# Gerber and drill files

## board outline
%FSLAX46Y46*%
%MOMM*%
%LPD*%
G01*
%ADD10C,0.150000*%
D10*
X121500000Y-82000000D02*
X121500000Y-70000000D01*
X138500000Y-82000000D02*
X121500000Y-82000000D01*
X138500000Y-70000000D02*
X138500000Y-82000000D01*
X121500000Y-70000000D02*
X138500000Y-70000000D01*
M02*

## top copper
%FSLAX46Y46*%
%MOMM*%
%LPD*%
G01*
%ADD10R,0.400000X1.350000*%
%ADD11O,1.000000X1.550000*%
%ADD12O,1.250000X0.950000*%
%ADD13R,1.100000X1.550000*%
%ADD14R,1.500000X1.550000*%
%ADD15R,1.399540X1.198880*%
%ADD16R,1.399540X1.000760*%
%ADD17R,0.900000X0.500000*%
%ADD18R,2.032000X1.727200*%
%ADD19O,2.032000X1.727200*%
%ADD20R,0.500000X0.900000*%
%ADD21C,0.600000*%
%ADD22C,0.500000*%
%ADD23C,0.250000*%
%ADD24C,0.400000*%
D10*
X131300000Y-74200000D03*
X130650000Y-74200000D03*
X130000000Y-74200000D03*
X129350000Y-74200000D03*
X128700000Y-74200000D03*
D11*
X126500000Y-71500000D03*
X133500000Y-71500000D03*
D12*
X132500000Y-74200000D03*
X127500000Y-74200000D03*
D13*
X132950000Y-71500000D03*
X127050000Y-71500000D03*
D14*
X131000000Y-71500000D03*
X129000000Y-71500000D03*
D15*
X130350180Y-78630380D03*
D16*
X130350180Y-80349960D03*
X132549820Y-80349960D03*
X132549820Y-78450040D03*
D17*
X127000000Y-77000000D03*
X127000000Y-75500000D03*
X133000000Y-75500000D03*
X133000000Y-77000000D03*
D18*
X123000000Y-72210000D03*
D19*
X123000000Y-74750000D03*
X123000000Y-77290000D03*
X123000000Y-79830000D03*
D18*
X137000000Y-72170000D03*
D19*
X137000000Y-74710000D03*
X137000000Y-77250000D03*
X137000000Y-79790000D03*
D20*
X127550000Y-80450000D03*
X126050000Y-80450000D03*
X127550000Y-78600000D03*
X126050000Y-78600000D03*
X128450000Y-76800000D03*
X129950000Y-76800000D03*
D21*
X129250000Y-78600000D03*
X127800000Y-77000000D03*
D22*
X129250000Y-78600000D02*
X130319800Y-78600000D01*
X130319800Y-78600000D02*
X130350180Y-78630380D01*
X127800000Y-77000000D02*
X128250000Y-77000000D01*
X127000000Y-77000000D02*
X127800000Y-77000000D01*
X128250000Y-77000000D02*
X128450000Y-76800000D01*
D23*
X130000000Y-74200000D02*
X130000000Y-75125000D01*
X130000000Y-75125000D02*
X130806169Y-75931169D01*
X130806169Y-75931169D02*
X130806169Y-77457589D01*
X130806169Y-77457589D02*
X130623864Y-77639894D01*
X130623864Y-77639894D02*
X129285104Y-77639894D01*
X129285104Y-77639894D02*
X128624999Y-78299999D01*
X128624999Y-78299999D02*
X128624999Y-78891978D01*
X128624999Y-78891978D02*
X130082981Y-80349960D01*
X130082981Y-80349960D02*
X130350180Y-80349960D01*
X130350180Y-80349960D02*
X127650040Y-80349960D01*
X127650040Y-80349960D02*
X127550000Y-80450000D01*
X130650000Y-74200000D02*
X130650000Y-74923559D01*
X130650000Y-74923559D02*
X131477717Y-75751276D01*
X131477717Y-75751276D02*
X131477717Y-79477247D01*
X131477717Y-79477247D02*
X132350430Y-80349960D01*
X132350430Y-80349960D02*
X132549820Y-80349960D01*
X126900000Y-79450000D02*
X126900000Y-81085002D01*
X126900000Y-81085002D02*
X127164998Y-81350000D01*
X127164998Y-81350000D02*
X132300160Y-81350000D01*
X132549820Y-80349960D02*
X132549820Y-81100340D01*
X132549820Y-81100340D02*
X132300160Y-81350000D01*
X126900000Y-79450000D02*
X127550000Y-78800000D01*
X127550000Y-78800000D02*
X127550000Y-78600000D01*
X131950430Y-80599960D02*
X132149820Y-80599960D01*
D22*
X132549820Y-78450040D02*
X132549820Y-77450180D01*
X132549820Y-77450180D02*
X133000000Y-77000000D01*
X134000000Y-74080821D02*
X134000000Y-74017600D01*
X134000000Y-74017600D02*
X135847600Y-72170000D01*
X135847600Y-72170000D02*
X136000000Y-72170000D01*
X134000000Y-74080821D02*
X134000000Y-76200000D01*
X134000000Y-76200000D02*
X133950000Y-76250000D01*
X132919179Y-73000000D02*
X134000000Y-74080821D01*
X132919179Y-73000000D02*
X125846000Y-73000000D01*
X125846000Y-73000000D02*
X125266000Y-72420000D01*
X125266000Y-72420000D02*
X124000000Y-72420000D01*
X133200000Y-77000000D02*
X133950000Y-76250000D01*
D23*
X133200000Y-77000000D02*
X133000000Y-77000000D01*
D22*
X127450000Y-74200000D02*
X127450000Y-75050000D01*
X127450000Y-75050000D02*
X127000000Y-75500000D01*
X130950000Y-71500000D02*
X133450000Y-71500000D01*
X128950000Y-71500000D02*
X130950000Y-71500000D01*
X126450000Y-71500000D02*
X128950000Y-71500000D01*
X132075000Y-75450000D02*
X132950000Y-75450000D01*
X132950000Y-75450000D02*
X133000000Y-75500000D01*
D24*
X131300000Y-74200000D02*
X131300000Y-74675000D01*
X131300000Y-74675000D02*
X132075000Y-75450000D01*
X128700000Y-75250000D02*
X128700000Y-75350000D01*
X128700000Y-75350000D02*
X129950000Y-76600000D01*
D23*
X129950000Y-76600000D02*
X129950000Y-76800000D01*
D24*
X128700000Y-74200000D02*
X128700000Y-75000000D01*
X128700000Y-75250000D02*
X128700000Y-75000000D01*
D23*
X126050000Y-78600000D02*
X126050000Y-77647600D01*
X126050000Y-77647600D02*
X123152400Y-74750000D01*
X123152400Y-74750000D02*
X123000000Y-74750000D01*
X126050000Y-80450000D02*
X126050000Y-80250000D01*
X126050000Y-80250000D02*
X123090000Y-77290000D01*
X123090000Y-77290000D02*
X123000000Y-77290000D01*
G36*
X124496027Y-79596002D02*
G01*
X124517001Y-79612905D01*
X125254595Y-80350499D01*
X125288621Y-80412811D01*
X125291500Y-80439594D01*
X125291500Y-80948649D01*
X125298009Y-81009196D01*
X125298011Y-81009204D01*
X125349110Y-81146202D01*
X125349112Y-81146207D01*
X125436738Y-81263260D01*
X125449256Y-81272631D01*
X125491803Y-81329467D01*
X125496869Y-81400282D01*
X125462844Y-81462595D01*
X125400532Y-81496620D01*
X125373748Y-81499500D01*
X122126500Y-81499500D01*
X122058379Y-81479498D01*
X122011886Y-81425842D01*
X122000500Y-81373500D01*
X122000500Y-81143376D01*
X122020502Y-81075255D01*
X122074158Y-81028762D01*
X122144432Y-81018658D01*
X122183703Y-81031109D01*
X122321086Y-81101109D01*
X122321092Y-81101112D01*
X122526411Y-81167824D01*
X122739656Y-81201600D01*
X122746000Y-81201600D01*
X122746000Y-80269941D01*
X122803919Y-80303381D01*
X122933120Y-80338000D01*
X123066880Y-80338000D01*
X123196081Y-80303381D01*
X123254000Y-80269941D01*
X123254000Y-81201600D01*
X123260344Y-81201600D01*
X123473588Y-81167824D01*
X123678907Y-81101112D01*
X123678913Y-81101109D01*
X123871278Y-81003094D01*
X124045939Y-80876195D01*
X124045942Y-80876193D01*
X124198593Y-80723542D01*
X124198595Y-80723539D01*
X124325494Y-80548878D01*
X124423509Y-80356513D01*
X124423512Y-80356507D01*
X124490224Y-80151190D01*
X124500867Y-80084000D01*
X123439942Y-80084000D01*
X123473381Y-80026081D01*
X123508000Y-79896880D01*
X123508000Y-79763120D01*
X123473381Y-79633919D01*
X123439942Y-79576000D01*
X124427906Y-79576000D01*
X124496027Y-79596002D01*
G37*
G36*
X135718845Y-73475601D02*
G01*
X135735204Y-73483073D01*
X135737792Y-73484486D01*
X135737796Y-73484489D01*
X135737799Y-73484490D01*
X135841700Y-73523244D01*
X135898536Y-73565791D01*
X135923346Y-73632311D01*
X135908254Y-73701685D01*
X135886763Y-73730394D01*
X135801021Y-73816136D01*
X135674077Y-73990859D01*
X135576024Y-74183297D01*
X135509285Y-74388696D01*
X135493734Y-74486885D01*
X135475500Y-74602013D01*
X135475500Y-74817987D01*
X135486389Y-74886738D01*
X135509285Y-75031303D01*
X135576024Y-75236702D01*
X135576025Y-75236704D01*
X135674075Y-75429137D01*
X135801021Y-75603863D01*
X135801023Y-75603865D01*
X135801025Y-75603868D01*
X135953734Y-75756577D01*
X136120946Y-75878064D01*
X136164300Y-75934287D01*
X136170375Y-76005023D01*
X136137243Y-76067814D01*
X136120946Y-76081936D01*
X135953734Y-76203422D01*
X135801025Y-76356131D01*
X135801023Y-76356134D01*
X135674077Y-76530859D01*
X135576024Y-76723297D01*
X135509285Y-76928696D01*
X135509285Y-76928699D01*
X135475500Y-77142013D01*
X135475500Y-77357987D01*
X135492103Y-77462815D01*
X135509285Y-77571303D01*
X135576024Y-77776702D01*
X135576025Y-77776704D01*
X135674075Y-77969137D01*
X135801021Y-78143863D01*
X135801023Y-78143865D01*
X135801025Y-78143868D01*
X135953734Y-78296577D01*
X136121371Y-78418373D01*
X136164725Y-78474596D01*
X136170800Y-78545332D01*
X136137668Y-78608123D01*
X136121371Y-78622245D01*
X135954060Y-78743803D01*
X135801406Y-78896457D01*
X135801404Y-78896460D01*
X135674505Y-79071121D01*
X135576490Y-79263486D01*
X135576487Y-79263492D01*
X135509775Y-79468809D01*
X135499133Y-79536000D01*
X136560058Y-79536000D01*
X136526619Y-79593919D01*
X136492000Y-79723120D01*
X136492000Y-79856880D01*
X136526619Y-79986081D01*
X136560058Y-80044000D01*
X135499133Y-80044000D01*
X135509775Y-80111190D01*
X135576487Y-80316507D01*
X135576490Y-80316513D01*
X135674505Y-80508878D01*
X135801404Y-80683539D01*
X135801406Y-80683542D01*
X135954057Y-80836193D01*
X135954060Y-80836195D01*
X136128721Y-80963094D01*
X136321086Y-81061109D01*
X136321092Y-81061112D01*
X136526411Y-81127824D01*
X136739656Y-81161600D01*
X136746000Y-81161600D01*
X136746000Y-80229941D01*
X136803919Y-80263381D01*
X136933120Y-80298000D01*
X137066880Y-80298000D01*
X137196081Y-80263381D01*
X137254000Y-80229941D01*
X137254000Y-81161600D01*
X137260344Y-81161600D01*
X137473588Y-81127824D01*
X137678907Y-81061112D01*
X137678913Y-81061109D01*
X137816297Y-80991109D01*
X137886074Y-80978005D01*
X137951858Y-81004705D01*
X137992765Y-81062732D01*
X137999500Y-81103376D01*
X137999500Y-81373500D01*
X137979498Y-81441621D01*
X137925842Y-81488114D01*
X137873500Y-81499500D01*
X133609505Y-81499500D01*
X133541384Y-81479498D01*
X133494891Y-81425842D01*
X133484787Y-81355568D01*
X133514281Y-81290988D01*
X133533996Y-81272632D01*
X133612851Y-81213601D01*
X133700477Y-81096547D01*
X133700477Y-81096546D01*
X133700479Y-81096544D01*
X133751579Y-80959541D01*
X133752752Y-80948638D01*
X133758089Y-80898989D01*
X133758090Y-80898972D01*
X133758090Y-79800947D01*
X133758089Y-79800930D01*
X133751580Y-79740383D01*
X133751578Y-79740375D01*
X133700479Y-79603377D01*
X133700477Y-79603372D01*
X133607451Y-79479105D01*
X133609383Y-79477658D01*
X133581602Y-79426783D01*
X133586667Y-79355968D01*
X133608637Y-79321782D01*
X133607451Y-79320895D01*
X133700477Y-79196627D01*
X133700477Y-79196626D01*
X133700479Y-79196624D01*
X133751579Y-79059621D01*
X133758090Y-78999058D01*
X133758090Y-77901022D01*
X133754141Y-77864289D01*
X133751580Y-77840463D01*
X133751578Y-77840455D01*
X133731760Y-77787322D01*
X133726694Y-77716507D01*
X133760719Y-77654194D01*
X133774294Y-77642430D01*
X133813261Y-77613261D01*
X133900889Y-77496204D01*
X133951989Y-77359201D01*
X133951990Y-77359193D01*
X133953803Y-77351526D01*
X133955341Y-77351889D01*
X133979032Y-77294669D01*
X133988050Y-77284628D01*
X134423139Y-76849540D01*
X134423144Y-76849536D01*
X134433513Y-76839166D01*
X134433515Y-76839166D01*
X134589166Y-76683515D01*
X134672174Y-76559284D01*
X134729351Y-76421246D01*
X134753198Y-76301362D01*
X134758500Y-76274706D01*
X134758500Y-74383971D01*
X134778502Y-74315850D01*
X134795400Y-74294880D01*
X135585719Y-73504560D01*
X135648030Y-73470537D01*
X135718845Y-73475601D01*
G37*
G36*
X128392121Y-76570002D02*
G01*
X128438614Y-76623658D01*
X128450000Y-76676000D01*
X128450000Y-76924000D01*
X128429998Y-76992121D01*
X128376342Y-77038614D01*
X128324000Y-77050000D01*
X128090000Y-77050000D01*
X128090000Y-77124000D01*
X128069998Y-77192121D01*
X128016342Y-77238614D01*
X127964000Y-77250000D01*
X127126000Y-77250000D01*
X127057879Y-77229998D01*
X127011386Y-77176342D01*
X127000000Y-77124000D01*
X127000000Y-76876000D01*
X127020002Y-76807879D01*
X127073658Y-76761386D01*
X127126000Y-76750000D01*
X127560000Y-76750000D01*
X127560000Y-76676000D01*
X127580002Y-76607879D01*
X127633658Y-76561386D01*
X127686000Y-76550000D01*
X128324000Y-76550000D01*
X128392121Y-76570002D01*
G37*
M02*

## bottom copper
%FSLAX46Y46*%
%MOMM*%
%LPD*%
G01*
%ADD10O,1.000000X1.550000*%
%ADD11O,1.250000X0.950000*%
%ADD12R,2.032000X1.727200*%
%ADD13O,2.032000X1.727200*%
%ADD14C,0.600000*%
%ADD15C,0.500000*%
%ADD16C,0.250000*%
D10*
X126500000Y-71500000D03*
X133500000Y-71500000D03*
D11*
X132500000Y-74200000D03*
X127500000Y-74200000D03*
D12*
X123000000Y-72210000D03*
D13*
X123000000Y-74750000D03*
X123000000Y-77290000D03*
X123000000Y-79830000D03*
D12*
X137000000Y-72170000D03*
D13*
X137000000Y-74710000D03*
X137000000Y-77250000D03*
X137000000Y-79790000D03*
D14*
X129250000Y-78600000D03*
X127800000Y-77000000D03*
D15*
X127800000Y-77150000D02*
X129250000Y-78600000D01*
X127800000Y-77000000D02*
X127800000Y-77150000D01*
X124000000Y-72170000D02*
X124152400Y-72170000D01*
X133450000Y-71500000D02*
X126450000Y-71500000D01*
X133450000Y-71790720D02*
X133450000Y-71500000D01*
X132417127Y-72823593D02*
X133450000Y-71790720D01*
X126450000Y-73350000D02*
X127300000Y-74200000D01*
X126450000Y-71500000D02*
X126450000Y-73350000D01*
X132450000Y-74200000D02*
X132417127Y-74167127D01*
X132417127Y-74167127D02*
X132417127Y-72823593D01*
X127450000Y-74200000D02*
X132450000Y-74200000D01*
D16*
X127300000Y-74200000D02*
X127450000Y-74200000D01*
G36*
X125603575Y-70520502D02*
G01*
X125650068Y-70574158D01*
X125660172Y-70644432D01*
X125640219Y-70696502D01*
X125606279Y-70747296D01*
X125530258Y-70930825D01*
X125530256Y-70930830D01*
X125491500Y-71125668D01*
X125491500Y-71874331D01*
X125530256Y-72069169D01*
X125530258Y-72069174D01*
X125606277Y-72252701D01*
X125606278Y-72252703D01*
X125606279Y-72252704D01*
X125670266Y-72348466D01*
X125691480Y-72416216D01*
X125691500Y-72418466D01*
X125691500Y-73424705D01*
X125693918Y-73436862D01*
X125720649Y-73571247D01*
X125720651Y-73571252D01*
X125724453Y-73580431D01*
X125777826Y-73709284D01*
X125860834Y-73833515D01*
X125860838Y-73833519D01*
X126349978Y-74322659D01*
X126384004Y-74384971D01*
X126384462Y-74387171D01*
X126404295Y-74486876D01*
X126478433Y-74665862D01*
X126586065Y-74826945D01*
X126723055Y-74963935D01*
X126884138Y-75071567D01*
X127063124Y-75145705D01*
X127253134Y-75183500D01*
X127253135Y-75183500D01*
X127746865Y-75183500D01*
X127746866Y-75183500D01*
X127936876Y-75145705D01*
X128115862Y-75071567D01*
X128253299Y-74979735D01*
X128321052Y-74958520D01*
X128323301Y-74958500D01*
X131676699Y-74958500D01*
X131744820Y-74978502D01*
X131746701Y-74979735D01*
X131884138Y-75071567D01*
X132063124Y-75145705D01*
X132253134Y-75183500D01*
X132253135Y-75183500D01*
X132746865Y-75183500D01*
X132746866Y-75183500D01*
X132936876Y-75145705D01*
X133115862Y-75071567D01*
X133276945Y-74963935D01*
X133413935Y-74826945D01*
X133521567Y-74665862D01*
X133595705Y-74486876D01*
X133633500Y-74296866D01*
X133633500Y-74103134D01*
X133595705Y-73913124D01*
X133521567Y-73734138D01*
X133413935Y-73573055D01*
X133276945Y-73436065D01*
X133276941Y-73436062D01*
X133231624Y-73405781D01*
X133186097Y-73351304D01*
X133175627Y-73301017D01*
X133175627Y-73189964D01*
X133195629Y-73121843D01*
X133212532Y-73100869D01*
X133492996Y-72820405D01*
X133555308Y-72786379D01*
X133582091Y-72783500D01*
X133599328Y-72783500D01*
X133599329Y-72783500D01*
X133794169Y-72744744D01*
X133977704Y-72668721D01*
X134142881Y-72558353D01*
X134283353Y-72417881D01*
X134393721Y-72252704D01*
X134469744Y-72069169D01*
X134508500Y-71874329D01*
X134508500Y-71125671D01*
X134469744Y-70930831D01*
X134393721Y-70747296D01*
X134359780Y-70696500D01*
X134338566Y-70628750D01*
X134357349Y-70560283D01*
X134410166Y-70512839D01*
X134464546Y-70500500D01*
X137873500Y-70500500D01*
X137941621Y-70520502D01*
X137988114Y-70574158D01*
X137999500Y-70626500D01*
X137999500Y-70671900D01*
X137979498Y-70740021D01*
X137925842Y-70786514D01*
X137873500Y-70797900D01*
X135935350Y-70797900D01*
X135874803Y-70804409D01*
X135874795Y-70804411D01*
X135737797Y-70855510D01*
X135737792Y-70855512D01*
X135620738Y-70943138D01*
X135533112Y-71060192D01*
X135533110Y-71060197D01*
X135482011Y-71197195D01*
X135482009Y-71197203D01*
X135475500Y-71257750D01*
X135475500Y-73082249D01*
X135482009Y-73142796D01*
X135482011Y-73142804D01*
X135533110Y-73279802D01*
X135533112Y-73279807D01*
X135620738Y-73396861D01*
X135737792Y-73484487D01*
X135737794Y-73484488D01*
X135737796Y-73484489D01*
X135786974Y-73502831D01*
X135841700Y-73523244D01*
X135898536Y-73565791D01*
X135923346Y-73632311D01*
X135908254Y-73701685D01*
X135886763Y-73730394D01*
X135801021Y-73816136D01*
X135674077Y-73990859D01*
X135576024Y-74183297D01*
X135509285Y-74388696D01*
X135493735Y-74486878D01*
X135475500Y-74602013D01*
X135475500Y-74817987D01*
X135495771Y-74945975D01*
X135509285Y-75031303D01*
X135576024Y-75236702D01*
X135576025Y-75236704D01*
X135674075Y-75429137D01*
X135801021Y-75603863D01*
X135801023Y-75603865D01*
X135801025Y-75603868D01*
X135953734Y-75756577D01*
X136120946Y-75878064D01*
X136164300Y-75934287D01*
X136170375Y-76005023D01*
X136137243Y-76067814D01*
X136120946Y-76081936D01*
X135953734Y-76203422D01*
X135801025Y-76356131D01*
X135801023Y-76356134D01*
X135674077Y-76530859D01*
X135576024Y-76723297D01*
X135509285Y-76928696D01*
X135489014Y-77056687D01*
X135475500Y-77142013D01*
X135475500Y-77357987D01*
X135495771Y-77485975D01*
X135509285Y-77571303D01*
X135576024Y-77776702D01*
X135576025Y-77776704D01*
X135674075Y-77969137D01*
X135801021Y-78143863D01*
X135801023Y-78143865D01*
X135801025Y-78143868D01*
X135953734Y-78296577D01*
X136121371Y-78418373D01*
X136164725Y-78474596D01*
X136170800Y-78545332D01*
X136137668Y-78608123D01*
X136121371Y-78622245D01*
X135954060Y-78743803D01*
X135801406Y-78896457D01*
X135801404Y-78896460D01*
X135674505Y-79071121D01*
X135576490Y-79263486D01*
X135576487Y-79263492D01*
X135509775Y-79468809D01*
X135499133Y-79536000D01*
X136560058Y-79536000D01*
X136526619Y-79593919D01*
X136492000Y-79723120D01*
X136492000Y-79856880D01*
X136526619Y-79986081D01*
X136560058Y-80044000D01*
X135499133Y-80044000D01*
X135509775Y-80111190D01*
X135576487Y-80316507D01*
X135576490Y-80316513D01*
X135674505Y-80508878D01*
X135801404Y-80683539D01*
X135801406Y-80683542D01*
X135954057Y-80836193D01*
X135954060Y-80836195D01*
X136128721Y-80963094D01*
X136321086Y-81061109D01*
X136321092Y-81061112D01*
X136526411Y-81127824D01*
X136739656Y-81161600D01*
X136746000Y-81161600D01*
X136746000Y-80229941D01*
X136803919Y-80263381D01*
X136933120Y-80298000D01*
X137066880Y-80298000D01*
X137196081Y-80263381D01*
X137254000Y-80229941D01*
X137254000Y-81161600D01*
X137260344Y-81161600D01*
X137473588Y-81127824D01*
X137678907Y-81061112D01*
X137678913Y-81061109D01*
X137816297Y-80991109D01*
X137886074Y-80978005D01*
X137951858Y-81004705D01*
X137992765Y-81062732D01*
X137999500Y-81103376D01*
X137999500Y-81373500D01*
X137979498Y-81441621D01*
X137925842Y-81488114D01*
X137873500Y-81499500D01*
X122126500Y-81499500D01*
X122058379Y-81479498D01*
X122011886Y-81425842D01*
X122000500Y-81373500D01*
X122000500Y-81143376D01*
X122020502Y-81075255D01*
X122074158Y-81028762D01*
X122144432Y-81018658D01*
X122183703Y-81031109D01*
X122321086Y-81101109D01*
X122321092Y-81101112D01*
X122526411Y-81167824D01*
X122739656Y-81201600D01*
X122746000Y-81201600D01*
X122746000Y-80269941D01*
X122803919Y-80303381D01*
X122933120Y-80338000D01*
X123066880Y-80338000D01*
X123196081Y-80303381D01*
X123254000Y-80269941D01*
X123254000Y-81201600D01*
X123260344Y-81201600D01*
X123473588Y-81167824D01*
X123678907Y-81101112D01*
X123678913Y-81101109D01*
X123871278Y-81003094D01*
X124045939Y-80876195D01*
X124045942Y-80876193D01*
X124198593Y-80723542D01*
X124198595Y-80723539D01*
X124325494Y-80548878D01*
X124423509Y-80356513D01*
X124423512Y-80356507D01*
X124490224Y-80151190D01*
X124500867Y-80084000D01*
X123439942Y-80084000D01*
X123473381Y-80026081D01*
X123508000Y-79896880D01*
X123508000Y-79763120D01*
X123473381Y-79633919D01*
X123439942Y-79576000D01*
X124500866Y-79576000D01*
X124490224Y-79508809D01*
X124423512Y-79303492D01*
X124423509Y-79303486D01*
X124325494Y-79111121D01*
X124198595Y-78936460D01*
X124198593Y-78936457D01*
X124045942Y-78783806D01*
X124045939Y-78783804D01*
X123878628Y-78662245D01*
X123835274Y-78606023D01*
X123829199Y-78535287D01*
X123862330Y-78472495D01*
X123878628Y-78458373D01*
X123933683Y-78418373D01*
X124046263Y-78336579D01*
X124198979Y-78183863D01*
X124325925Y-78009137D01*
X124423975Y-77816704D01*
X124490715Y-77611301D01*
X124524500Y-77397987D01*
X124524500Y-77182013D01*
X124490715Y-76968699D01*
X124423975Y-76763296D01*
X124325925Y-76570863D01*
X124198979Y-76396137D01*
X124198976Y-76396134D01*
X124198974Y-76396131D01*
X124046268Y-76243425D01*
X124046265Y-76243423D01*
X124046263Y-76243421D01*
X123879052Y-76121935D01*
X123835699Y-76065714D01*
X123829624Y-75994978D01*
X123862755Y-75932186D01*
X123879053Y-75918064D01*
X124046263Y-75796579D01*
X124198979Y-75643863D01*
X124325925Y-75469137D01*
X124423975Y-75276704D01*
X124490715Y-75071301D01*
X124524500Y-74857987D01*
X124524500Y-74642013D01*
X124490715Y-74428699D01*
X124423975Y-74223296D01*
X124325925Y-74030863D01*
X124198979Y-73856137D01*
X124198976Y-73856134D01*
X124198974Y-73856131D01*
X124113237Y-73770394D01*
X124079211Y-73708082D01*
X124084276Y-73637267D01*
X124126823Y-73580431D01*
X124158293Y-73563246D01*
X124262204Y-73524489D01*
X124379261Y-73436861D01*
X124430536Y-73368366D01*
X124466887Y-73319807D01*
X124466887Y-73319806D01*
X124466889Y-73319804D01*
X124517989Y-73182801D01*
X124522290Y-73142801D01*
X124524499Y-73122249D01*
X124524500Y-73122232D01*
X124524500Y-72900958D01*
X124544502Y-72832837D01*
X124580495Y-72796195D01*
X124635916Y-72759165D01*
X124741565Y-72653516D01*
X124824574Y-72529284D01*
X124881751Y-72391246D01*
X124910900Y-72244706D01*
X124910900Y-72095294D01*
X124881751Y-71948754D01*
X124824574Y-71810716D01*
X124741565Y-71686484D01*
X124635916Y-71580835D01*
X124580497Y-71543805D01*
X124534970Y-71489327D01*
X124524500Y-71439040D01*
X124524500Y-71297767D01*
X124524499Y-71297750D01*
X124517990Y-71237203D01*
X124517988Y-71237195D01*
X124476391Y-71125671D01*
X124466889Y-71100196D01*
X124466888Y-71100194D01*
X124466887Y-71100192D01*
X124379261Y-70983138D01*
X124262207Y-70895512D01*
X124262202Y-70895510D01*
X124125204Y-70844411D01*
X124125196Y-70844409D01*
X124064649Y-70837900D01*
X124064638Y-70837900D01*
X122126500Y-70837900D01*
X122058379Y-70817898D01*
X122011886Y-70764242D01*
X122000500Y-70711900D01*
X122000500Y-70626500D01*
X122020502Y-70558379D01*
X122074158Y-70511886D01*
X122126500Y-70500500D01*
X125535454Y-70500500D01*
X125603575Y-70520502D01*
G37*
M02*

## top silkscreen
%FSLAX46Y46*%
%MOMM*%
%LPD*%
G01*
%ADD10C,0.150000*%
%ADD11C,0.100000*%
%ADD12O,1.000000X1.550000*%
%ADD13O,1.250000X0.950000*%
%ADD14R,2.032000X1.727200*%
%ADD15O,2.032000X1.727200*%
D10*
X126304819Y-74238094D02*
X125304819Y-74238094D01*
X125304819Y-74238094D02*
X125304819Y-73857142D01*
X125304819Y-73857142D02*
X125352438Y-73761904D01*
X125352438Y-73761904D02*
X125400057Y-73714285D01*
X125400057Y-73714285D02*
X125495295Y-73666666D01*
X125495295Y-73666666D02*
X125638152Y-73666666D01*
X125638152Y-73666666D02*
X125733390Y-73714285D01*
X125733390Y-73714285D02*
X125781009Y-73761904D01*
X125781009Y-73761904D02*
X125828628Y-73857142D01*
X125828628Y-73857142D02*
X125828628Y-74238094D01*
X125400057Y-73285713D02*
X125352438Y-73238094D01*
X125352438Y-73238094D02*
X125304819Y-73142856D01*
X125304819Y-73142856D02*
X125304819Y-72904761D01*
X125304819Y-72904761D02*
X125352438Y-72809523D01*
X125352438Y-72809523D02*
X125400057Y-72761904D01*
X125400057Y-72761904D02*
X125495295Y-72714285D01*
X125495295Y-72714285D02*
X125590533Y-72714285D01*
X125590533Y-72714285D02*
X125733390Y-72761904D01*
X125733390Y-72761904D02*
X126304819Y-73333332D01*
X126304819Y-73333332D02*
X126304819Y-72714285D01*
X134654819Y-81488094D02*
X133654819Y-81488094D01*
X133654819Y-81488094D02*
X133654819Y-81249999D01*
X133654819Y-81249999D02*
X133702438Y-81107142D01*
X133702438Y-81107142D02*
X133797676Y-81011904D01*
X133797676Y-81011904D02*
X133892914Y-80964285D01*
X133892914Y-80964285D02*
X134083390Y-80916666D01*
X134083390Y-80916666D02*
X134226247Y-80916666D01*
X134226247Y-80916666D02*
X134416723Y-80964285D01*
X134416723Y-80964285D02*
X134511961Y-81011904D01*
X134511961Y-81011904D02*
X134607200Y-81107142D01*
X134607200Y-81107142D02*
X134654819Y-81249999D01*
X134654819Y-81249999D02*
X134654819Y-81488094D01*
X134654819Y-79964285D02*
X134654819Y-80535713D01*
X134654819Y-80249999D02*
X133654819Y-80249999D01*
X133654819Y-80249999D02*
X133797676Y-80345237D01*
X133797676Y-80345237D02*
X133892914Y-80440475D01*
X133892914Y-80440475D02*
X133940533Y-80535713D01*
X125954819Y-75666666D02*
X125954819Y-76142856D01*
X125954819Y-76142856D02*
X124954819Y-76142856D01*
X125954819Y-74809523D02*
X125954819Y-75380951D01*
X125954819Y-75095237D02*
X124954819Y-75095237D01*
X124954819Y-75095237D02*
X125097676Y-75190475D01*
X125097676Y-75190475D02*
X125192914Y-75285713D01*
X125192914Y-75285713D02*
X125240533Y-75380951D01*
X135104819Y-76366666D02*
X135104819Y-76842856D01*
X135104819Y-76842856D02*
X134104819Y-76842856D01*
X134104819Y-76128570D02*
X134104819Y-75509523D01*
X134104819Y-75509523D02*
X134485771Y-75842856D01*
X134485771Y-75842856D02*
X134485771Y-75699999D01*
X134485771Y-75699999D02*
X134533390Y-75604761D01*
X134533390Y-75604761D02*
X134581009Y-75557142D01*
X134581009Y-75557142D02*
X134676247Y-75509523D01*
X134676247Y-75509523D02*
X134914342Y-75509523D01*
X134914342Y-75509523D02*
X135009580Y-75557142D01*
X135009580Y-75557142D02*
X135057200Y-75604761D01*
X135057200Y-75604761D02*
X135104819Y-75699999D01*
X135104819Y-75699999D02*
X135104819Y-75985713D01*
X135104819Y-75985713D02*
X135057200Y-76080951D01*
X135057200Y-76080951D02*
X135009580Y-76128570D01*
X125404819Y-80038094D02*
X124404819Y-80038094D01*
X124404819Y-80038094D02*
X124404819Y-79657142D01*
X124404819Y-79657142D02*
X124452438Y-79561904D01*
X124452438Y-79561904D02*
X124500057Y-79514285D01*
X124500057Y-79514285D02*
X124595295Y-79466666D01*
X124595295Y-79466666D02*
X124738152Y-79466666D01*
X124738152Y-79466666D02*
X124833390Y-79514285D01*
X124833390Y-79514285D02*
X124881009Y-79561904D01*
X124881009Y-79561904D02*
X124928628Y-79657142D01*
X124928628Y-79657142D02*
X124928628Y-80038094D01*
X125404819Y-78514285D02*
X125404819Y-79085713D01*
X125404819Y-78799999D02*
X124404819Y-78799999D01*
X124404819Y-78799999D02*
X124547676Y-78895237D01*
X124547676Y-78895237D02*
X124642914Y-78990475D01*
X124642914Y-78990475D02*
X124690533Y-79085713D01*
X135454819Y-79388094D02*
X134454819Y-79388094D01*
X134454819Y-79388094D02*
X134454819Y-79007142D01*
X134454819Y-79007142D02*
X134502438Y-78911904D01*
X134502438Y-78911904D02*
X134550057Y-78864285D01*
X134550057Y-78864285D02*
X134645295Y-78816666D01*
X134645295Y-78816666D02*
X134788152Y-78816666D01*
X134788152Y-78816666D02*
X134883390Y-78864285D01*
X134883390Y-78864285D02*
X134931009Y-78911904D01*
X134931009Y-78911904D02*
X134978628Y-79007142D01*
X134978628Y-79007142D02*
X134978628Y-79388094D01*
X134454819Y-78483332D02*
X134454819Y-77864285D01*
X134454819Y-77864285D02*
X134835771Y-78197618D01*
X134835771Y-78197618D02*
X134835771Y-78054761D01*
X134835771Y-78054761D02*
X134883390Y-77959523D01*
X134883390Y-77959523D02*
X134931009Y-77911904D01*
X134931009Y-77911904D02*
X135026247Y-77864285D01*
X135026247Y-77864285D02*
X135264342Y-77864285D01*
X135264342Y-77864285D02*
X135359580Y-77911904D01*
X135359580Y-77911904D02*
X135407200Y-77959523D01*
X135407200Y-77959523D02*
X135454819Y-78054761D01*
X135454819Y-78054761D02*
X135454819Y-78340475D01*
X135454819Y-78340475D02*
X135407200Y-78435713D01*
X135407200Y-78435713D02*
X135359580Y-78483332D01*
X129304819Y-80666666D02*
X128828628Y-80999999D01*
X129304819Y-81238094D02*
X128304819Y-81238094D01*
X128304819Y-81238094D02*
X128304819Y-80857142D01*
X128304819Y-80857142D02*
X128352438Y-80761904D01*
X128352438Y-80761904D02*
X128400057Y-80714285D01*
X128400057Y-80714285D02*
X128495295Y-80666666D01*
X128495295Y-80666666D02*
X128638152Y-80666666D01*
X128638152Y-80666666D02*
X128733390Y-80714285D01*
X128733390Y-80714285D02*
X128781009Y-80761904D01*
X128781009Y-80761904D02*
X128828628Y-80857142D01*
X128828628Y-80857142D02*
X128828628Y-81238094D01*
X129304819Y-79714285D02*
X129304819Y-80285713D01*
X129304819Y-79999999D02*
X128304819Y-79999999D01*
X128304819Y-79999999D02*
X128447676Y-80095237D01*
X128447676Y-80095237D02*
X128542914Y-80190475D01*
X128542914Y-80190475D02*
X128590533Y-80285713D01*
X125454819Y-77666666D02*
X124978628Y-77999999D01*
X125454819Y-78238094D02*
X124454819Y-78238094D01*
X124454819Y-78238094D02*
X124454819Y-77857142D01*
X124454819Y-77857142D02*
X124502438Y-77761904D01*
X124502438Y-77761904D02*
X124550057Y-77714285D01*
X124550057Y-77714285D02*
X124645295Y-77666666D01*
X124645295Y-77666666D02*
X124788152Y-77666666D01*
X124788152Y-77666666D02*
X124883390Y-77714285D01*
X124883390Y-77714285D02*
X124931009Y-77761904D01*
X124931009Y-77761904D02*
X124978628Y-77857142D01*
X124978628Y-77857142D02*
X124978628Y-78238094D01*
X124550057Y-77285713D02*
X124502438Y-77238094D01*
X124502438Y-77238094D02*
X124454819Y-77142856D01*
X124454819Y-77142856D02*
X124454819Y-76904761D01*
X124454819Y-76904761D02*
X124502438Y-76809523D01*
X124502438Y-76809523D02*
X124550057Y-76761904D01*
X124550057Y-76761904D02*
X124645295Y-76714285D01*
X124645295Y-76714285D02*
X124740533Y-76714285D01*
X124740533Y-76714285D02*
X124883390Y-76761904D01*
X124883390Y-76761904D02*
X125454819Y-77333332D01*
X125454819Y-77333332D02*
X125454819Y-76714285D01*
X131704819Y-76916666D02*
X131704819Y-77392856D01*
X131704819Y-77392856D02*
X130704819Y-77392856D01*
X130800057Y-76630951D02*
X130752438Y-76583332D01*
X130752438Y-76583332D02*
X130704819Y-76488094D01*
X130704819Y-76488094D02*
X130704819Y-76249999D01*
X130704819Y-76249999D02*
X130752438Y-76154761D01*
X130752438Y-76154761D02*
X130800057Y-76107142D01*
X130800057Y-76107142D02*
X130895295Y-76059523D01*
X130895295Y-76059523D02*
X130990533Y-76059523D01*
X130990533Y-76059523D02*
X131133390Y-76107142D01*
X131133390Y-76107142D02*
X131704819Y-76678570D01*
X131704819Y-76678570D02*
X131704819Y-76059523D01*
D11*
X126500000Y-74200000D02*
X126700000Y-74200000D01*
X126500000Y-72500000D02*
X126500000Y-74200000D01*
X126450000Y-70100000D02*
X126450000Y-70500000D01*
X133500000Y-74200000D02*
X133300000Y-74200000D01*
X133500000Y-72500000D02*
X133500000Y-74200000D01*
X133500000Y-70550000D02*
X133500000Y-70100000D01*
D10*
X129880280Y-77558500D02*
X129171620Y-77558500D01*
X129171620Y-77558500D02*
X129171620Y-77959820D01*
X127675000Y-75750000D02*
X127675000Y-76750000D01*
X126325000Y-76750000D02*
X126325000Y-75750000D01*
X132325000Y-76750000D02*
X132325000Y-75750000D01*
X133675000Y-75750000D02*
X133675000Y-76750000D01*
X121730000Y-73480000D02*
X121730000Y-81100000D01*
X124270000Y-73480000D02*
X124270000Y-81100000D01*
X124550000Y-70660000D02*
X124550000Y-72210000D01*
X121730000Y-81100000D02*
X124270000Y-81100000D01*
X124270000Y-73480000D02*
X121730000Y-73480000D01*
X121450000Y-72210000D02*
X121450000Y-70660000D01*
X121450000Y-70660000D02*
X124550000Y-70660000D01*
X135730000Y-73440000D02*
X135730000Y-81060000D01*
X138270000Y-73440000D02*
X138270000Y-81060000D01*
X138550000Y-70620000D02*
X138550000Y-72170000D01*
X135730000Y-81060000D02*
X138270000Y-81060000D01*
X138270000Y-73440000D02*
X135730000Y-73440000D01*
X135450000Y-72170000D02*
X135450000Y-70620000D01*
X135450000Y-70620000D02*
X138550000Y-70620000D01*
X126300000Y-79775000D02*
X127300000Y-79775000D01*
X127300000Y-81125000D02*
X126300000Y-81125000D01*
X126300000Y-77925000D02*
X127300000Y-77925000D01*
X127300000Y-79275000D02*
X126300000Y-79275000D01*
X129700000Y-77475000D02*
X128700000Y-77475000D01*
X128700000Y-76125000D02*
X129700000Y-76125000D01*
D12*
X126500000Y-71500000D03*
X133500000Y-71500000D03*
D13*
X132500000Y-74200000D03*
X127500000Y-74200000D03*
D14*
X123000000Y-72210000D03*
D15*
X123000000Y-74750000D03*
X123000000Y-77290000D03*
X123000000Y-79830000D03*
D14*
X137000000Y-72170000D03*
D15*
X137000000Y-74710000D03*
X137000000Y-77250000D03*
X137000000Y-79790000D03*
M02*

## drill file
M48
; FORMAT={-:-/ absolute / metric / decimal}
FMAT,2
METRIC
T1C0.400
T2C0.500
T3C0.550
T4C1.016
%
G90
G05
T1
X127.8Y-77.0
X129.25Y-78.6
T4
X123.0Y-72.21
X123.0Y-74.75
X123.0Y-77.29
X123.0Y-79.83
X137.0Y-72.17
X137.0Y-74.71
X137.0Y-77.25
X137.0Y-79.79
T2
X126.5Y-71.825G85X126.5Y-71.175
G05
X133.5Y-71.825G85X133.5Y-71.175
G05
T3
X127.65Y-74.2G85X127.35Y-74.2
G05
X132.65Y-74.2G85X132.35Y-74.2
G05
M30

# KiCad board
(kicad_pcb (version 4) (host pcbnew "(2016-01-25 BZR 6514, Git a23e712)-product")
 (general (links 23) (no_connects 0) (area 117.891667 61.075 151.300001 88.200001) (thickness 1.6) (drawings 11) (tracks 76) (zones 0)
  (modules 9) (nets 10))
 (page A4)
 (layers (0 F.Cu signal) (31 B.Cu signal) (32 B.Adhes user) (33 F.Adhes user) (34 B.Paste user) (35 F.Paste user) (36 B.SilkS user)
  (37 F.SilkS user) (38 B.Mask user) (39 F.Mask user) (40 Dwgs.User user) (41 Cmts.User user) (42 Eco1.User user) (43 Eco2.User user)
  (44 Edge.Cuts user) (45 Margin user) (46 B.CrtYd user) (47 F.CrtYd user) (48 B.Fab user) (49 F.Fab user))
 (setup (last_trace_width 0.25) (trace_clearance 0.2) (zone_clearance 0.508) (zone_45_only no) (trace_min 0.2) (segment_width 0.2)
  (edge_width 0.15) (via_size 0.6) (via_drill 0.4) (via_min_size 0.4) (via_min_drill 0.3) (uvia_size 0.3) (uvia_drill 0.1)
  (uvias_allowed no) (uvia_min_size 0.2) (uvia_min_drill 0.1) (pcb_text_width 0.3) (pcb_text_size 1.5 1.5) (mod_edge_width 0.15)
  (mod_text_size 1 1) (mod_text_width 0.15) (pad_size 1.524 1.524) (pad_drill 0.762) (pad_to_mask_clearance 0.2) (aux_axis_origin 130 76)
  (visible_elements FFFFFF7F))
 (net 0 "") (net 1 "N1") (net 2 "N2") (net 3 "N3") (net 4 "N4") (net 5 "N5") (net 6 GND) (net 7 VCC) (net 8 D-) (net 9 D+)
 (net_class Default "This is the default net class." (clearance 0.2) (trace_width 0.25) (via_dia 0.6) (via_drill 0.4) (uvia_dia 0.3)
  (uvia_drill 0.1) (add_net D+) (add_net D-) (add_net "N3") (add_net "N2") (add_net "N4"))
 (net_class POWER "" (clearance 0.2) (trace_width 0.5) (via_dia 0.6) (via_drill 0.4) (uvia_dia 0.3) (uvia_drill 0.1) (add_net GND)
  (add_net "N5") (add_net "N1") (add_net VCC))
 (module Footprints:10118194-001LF (layer F.Cu) (at 130 71.5 180)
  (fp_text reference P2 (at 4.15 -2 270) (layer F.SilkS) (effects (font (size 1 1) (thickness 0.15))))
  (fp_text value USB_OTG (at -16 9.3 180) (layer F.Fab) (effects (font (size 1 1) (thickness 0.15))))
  (fp_line (start 3.5 -2.7) (end 3.3 -2.7) (layer F.SilkS) (width 0.1))
  (fp_line (start 3.5 -1) (end 3.5 -2.7) (layer F.SilkS) (width 0.1))
  (fp_line (start 3.55 1.4) (end 3.55 1) (layer F.SilkS) (width 0.1))
  (fp_line (start -3.5 -2.7) (end -3.3 -2.7) (layer F.SilkS) (width 0.1))
  (fp_line (start -3.5 -1) (end -3.5 -2.7) (layer F.SilkS) (width 0.1))
  (fp_line (start -3.5 0.95) (end -3.5 1.4) (layer F.SilkS) (width 0.1))
  (pad 1 smd rect (at -1.3 -2.7 180) (size 0.4 1.35) (layers F.Cu F.Paste F.Mask) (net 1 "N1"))
  (pad 2 smd rect (at -0.65 -2.7 180) (size 0.4 1.35) (layers F.Cu F.Paste F.Mask) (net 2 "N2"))
  (pad 3 smd rect (at 0 -2.7 180) (size 0.4 1.35) (layers F.Cu F.Paste F.Mask) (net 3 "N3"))
  (pad 4 smd rect (at 0.65 -2.7 180) (size 0.4 1.35) (layers F.Cu F.Paste F.Mask))
  (pad 5 smd rect (at 1.3 -2.7 180) (size 0.4 1.35) (layers F.Cu F.Paste F.Mask) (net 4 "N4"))
  (pad 6 thru_hole oval (at 3.5 0 180) (size 1 1.55) (drill oval 0.5 1.15) (layers *.Cu *.Mask F.SilkS) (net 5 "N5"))
  (pad 6 thru_hole oval (at -3.5 0 180) (size 1 1.55) (drill oval 0.5 1.15) (layers *.Cu *.Mask F.SilkS) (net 5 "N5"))
  (pad 6 thru_hole oval (at -2.5 -2.7 180) (size 1.25 0.95) (drill oval 0.85 0.55) (layers *.Cu *.Mask F.SilkS) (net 5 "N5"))
  (pad 6 thru_hole oval (at 2.5 -2.7 180) (size 1.25 0.95) (drill oval 0.85 0.55) (layers *.Cu *.Mask F.SilkS) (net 5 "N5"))
  (pad 6 smd rect (at -2.95 0 270) (size 1.55 1.1) (layers F.Cu F.Paste F.Mask) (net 5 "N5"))
  (pad 6 smd rect (at 2.95 0 270) (size 1.55 1.1) (layers F.Cu F.Paste F.Mask) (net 5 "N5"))
  (pad 6 smd rect (at -1 0 270) (size 1.55 1.5) (layers F.Cu F.Paste F.Mask) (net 5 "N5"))
  (pad 6 smd rect (at 1 0 270) (size 1.55 1.5) (layers F.Cu F.Paste F.Mask) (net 5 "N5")))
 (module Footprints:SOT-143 (layer F.Cu) (at 131.45 79.4 270)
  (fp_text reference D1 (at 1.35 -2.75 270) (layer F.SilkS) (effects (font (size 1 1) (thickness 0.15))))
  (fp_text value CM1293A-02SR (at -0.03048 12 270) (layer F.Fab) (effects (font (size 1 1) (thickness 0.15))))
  (fp_line (start -1.8415 1.56972) (end -1.8415 2.27838) (layer F.SilkS) (width 0.15))
  (fp_line (start -1.8415 2.27838) (end -1.44018 2.27838) (layer F.SilkS) (width 0.15))
  (pad 1 smd rect (at -0.76962 1.09982 270) (size 1.19888 1.39954) (layers F.Cu F.Paste F.Mask) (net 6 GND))
  (pad 2 smd rect (at 0.94996 1.09982 270) (size 1.00076 1.39954) (layers F.Cu F.Paste F.Mask) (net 3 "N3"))
  (pad 3 smd rect (at 0.94996 -1.09982 270) (size 1.00076 1.39954) (layers F.Cu F.Paste F.Mask) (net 2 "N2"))
  (pad 4 smd rect (at -0.94996 -1.09982 270) (size 1.00076 1.39954) (layers F.Cu F.Paste F.Mask) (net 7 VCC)))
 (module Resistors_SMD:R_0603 (layer F.Cu) (at 127 76.25 90)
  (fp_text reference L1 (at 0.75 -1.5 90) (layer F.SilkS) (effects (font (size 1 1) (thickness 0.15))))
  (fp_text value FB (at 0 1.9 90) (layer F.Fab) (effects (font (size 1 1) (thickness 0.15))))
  (fp_line (start 0.5 0.675) (end -0.5 0.675) (layer F.SilkS) (width 0.15))
  (fp_line (start -0.5 -0.675) (end 0.5 -0.675) (layer F.SilkS) (width 0.15))
  (pad 1 smd rect (at -0.75 0 90) (size 0.5 0.9) (layers F.Cu F.Paste F.Mask) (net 6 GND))
  (pad 2 smd rect (at 0.75 0 90) (size 0.5 0.9) (layers F.Cu F.Paste F.Mask) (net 5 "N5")))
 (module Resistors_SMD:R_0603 (layer F.Cu) (at 133 76.25 270)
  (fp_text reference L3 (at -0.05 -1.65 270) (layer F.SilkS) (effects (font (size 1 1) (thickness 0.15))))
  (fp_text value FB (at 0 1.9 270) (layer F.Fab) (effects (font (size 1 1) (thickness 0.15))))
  (fp_line (start 0.5 0.675) (end -0.5 0.675) (layer F.SilkS) (width 0.15))
  (fp_line (start -0.5 -0.675) (end 0.5 -0.675) (layer F.SilkS) (width 0.15))
  (pad 1 smd rect (at -0.75 0 270) (size 0.5 0.9) (layers F.Cu F.Paste F.Mask) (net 1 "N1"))
  (pad 2 smd rect (at 0.75 0 270) (size 0.5 0.9) (layers F.Cu F.Paste F.Mask) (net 7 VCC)))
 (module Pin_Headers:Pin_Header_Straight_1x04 (layer F.Cu) (at 123 72.21)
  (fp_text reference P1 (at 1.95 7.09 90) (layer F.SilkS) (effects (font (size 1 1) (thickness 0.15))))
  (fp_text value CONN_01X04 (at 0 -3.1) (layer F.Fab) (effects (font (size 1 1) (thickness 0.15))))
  (fp_line (start -1.27 1.27) (end -1.27 8.89) (layer F.SilkS) (width 0.15))
  (fp_line (start 1.27 1.27) (end 1.27 8.89) (layer F.SilkS) (width 0.15))
  (fp_line (start 1.55 -1.55) (end 1.55 0) (layer F.SilkS) (width 0.15))
  (fp_line (start -1.27 8.89) (end 1.27 8.89) (layer F.SilkS) (width 0.15))
  (fp_line (start 1.27 1.27) (end -1.27 1.27) (layer F.SilkS) (width 0.15))
  (fp_line (start -1.55 0) (end -1.55 -1.55) (layer F.SilkS) (width 0.15))
  (fp_line (start -1.55 -1.55) (end 1.55 -1.55) (layer F.SilkS) (width 0.15))
  (pad 1 thru_hole rect (at 0 0) (size 2.032 1.7272) (drill 1.016) (layers *.Cu *.Mask F.SilkS) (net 7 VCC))
  (pad 2 thru_hole oval (at 0 2.54) (size 2.032 1.7272) (drill 1.016) (layers *.Cu *.Mask F.SilkS) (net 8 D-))
  (pad 3 thru_hole oval (at 0 5.08) (size 2.032 1.7272) (drill 1.016) (layers *.Cu *.Mask F.SilkS) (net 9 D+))
  (pad 4 thru_hole oval (at 0 7.62) (size 2.032 1.7272) (drill 1.016) (layers *.Cu *.Mask F.SilkS) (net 6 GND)))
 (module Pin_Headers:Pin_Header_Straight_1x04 (layer F.Cu) (at 137 72.17)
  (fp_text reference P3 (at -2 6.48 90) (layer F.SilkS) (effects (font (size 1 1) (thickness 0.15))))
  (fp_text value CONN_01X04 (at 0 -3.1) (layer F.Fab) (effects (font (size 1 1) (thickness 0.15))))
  (fp_line (start -1.27 1.27) (end -1.27 8.89) (layer F.SilkS) (width 0.15))
  (fp_line (start 1.27 1.27) (end 1.27 8.89) (layer F.SilkS) (width 0.15))
  (fp_line (start 1.55 -1.55) (end 1.55 0) (layer F.SilkS) (width 0.15))
  (fp_line (start -1.27 8.89) (end 1.27 8.89) (layer F.SilkS) (width 0.15))
  (fp_line (start 1.27 1.27) (end -1.27 1.27) (layer F.SilkS) (width 0.15))
  (fp_line (start -1.55 0) (end -1.55 -1.55) (layer F.SilkS) (width 0.15))
  (fp_line (start -1.55 -1.55) (end 1.55 -1.55) (layer F.SilkS) (width 0.15))
  (pad 1 thru_hole rect (at 0 0) (size 2.032 1.7272) (drill 1.016) (layers *.Cu *.Mask F.SilkS) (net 7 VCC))
  (pad 2 thru_hole oval (at 0 2.54) (size 2.032 1.7272) (drill 1.016) (layers *.Cu *.Mask F.SilkS))
  (pad 3 thru_hole oval (at 0 5.08) (size 2.032 1.7272) (drill 1.016) (layers *.Cu *.Mask F.SilkS))
  (pad 4 thru_hole oval (at 0 7.62) (size 2.032 1.7272) (drill 1.016) (layers *.Cu *.Mask F.SilkS) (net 6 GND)))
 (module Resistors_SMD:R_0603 (layer F.Cu) (at 126.8 80.45 180)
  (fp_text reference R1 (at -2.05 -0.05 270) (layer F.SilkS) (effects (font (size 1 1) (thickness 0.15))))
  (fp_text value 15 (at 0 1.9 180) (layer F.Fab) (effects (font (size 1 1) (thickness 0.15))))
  (fp_line (start 0.5 0.675) (end -0.5 0.675) (layer F.SilkS) (width 0.15))
  (fp_line (start -0.5 -0.675) (end 0.5 -0.675) (layer F.SilkS) (width 0.15))
  (pad 1 smd rect (at -0.75 0 180) (size 0.5 0.9) (layers F.Cu F.Paste F.Mask) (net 3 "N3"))
  (pad 2 smd rect (at 0.75 0 180) (size 0.5 0.9) (layers F.Cu F.Paste F.Mask) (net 9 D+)))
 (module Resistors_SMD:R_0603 (layer F.Cu) (at 126.8 78.6 180)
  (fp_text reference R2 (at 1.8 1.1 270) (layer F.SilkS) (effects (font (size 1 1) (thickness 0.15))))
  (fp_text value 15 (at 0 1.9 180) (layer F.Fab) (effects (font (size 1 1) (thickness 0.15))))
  (fp_line (start 0.5 0.675) (end -0.5 0.675) (layer F.SilkS) (width 0.15))
  (fp_line (start -0.5 -0.675) (end 0.5 -0.675) (layer F.SilkS) (width 0.15))
  (pad 1 smd rect (at -0.75 0 180) (size 0.5 0.9) (layers F.Cu F.Paste F.Mask) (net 2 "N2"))
  (pad 2 smd rect (at 0.75 0 180) (size 0.5 0.9) (layers F.Cu F.Paste F.Mask) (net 8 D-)))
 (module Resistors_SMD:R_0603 (layer F.Cu) (at 129.2 76.8)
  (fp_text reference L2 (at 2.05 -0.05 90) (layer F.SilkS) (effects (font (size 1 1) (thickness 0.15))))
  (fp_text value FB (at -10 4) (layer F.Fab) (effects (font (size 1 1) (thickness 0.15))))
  (fp_line (start 0.5 0.675) (end -0.5 0.675) (layer F.SilkS) (width 0.15))
  (fp_line (start -0.5 -0.675) (end 0.5 -0.675) (layer F.SilkS) (width 0.15))
  (pad 1 smd rect (at -0.75 0) (size 0.5 0.9) (layers F.Cu F.Paste F.Mask) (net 6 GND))
  (pad 2 smd rect (at 0.75 0) (size 0.5 0.9) (layers F.Cu F.Paste F.Mask) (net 4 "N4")))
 (gr_line (start 121.5 82) (end 121.5 70) (layer Edge.Cuts) (width 0.15))
 (gr_line (start 138.5 82) (end 121.5 82) (layer Edge.Cuts) (width 0.15))
 (gr_line (start 138.5 70) (end 138.5 82) (layer Edge.Cuts) (width 0.15))
 (gr_line (start 121.5 70) (end 138.5 70) (layer Edge.Cuts) (width 0.15))
 (segment (start 129.25 78.6) (end 130.3198 78.6) (width 0.5) (layer F.Cu) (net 6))
 (segment (start 130.3198 78.6) (end 130.35018 78.63038) (width 0.5) (layer F.Cu) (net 6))
 (segment (start 127.8 77.15) (end 129.25 78.6) (width 0.5) (layer B.Cu) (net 6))
 (via (at 129.25 78.6) (size 0.6) (drill 0.4) (layers F.Cu B.Cu) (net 6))
 (segment (start 127.8 77) (end 127.8 77.15) (width 0.5) (layer B.Cu) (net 6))
 (segment (start 127.8 77) (end 128.25 77) (width 0.5) (layer F.Cu) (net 6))
 (segment (start 127 77) (end 127.8 77) (width 0.5) (layer F.Cu) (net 6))
 (via (at 127.8 77) (size 0.6) (drill 0.4) (layers F.Cu B.Cu) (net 6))
 (segment (start 128.25 77) (end 128.45 76.8) (width 0.5) (layer F.Cu) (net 6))
 (segment (start 130 74.2) (end 130 75.125) (width 0.25) (layer F.Cu) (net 3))
 (segment (start 130 75.125) (end 130.806169 75.931169) (width 0.25) (layer F.Cu) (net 3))
 (segment (start 130.806169 75.931169) (end 130.806169 77.457589) (width 0.25) (layer F.Cu) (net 3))
 (segment (start 130.806169 77.457589) (end 130.623864 77.639894) (width 0.25) (layer F.Cu) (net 3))
 (segment (start 130.623864 77.639894) (end 129.285104 77.639894) (width 0.25) (layer F.Cu) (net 3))
 (segment (start 129.285104 77.639894) (end 128.624999 78.299999) (width 0.25) (layer F.Cu) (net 3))
 (segment (start 128.624999 78.299999) (end 128.624999 78.891978) (width 0.25) (layer F.Cu) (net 3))
 (segment (start 128.624999 78.891978) (end 130.082981 80.34996) (width 0.25) (layer F.Cu) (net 3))
 (segment (start 130.082981 80.34996) (end 130.35018 80.34996) (width 0.25) (layer F.Cu) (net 3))
 (segment (start 130.35018 80.34996) (end 127.65004 80.34996) (width 0.25) (layer F.Cu) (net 3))
 (segment (start 127.65004 80.34996) (end 127.55 80.45) (width 0.25) (layer F.Cu) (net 3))
 (segment (start 130.65 74.2) (end 130.65 74.923559) (width 0.25) (layer F.Cu) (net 2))
 (segment (start 130.65 74.923559) (end 131.477717 75.751276) (width 0.25) (layer F.Cu) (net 2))
 (segment (start 131.477717 75.751276) (end 131.477717 79.477247) (width 0.25) (layer F.Cu) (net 2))
 (segment (start 131.477717 79.477247) (end 132.35043 80.34996) (width 0.25) (layer F.Cu) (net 2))
 (segment (start 132.35043 80.34996) (end 132.54982 80.34996) (width 0.25) (layer F.Cu) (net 2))
 (segment (start 126.9 79.45) (end 126.9 81.085002) (width 0.25) (layer F.Cu) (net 2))
 (segment (start 126.9 81.085002) (end 127.164998 81.35) (width 0.25) (layer F.Cu) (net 2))
 (segment (start 127.164998 81.35) (end 132.30016 81.35) (width 0.25) (layer F.Cu) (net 2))
 (segment (start 132.54982 80.34996) (end 132.54982 81.10034) (width 0.25) (layer F.Cu) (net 2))
 (segment (start 132.54982 81.10034) (end 132.30016 81.35) (width 0.25) (layer F.Cu) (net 2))
 (segment (start 126.9 79.45) (end 127.55 78.8) (width 0.25) (layer F.Cu) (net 2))
 (segment (start 127.55 78.8) (end 127.55 78.6) (width 0.25) (layer F.Cu) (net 2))
 (segment (start 131.95043 80.59996) (end 132.14982 80.59996) (width 0.25) (layer F.Cu) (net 2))
 (segment (start 132.54982 78.45004) (end 132.54982 77.45018) (width 0.5) (layer F.Cu) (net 7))
 (segment (start 132.54982 77.45018) (end 133 77) (width 0.5) (layer F.Cu) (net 7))
 (segment (start 124 72.17) (end 124.1524 72.17) (width 0.5) (layer B.Cu) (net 7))
 (segment (start 134 74.080821) (end 134 74.0176) (width 0.5) (layer F.Cu) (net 7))
 (segment (start 134 74.0176) (end 135.8476 72.17) (width 0.5) (layer F.Cu) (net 7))
 (segment (start 135.8476 72.17) (end 136 72.17) (width 0.5) (layer F.Cu) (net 7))
 (segment (start 134 74.080821) (end 134 76.2) (width 0.5) (layer F.Cu) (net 7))
 (segment (start 134 76.2) (end 133.95 76.25) (width 0.5) (layer F.Cu) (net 7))
 (segment (start 132.919179 73) (end 134 74.080821) (width 0.5) (layer F.Cu) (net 7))
 (segment (start 132.919179 73) (end 125.846 73) (width 0.5) (layer F.Cu) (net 7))
 (segment (start 125.846 73) (end 125.266 72.42) (width 0.5) (layer F.Cu) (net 7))
 (segment (start 125.266 72.42) (end 124 72.42) (width 0.5) (layer F.Cu) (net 7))
 (segment (start 133.2 77) (end 133.95 76.25) (width 0.5) (layer F.Cu) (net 7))
 (segment (start 133.2 77) (end 133 77) (width 0.25) (layer F.Cu) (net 7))
 (segment (start 133.45 71.5) (end 126.45 71.5) (width 0.5) (layer B.Cu) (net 5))
 (segment (start 133.45 71.79072) (end 133.45 71.5) (width 0.5) (layer B.Cu) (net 5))
 (segment (start 132.417127 72.823593) (end 133.45 71.79072) (width 0.5) (layer B.Cu) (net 5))
 (segment (start 126.45 73.35) (end 127.3 74.2) (width 0.5) (layer B.Cu) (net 5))
 (segment (start 126.45 71.5) (end 126.45 73.35) (width 0.5) (layer B.Cu) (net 5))
 (segment (start 132.45 74.2) (end 132.417127 74.167127) (width 0.5) (layer B.Cu) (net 5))
 (segment (start 132.417127 74.167127) (end 132.417127 72.823593) (width 0.5) (layer B.Cu) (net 5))
 (segment (start 127.45 74.2) (end 132.45 74.2) (width 0.5) (layer B.Cu) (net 5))
 (segment (start 127.45 74.2) (end 127.45 75.05) (width 0.5) (layer F.Cu) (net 5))
 (segment (start 127.45 75.05) (end 127 75.5) (width 0.5) (layer F.Cu) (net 5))
 (segment (start 130.95 71.5) (end 133.45 71.5) (width 0.5) (layer F.Cu) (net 5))
 (segment (start 128.95 71.5) (end 130.95 71.5) (width 0.5) (layer F.Cu) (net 5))
 (segment (start 126.45 71.5) (end 128.95 71.5) (width 0.5) (layer F.Cu) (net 5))
 (segment (start 127.3 74.2) (end 127.45 74.2) (width 0.25) (layer B.Cu) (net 5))
 (segment (start 132.075 75.45) (end 132.95 75.45) (width 0.5) (layer F.Cu) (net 1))
 (segment (start 132.95 75.45) (end 133 75.5) (width 0.5) (layer F.Cu) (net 1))
 (segment (start 131.3 74.2) (end 131.3 74.675) (width 0.4) (layer F.Cu) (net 1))
 (segment (start 131.3 74.675) (end 132.075 75.45) (width 0.4) (layer F.Cu) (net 1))
 (segment (start 128.7 75.25) (end 128.7 75.35) (width 0.4) (layer F.Cu) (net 4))
 (segment (start 128.7 75.35) (end 129.95 76.6) (width 0.4) (layer F.Cu) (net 4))
 (segment (start 129.95 76.6) (end 129.95 76.8) (width 0.25) (layer F.Cu) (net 4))
 (segment (start 128.7 74.2) (end 128.7 75) (width 0.4) (layer F.Cu) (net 4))
 (segment (start 128.7 75.25) (end 128.7 75) (width 0.4) (layer F.Cu) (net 4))
 (segment (start 126.05 78.6) (end 126.05 77.6476) (width 0.25) (layer F.Cu) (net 8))
 (segment (start 126.05 77.6476) (end 123.1524 74.75) (width 0.25) (layer F.Cu) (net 8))
 (segment (start 123.1524 74.75) (end 123 74.75) (width 0.25) (layer F.Cu) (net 8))
 (segment (start 126.05 80.45) (end 126.05 80.25) (width 0.25) (layer F.Cu) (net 9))
 (segment (start 126.05 80.25) (end 123.09 77.29) (width 0.25) (layer F.Cu) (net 9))
 (segment (start 123.09 77.29) (end 123 77.29) (width 0.25) (layer F.Cu) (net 9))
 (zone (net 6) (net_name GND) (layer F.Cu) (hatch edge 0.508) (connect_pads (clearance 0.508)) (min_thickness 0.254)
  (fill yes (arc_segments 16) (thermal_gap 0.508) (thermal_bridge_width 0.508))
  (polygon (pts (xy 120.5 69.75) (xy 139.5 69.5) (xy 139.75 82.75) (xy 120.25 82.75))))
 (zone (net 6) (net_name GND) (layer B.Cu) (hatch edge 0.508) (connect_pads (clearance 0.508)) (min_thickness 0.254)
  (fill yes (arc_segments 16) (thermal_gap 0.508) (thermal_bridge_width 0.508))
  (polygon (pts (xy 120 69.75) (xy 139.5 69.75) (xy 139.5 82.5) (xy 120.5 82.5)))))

